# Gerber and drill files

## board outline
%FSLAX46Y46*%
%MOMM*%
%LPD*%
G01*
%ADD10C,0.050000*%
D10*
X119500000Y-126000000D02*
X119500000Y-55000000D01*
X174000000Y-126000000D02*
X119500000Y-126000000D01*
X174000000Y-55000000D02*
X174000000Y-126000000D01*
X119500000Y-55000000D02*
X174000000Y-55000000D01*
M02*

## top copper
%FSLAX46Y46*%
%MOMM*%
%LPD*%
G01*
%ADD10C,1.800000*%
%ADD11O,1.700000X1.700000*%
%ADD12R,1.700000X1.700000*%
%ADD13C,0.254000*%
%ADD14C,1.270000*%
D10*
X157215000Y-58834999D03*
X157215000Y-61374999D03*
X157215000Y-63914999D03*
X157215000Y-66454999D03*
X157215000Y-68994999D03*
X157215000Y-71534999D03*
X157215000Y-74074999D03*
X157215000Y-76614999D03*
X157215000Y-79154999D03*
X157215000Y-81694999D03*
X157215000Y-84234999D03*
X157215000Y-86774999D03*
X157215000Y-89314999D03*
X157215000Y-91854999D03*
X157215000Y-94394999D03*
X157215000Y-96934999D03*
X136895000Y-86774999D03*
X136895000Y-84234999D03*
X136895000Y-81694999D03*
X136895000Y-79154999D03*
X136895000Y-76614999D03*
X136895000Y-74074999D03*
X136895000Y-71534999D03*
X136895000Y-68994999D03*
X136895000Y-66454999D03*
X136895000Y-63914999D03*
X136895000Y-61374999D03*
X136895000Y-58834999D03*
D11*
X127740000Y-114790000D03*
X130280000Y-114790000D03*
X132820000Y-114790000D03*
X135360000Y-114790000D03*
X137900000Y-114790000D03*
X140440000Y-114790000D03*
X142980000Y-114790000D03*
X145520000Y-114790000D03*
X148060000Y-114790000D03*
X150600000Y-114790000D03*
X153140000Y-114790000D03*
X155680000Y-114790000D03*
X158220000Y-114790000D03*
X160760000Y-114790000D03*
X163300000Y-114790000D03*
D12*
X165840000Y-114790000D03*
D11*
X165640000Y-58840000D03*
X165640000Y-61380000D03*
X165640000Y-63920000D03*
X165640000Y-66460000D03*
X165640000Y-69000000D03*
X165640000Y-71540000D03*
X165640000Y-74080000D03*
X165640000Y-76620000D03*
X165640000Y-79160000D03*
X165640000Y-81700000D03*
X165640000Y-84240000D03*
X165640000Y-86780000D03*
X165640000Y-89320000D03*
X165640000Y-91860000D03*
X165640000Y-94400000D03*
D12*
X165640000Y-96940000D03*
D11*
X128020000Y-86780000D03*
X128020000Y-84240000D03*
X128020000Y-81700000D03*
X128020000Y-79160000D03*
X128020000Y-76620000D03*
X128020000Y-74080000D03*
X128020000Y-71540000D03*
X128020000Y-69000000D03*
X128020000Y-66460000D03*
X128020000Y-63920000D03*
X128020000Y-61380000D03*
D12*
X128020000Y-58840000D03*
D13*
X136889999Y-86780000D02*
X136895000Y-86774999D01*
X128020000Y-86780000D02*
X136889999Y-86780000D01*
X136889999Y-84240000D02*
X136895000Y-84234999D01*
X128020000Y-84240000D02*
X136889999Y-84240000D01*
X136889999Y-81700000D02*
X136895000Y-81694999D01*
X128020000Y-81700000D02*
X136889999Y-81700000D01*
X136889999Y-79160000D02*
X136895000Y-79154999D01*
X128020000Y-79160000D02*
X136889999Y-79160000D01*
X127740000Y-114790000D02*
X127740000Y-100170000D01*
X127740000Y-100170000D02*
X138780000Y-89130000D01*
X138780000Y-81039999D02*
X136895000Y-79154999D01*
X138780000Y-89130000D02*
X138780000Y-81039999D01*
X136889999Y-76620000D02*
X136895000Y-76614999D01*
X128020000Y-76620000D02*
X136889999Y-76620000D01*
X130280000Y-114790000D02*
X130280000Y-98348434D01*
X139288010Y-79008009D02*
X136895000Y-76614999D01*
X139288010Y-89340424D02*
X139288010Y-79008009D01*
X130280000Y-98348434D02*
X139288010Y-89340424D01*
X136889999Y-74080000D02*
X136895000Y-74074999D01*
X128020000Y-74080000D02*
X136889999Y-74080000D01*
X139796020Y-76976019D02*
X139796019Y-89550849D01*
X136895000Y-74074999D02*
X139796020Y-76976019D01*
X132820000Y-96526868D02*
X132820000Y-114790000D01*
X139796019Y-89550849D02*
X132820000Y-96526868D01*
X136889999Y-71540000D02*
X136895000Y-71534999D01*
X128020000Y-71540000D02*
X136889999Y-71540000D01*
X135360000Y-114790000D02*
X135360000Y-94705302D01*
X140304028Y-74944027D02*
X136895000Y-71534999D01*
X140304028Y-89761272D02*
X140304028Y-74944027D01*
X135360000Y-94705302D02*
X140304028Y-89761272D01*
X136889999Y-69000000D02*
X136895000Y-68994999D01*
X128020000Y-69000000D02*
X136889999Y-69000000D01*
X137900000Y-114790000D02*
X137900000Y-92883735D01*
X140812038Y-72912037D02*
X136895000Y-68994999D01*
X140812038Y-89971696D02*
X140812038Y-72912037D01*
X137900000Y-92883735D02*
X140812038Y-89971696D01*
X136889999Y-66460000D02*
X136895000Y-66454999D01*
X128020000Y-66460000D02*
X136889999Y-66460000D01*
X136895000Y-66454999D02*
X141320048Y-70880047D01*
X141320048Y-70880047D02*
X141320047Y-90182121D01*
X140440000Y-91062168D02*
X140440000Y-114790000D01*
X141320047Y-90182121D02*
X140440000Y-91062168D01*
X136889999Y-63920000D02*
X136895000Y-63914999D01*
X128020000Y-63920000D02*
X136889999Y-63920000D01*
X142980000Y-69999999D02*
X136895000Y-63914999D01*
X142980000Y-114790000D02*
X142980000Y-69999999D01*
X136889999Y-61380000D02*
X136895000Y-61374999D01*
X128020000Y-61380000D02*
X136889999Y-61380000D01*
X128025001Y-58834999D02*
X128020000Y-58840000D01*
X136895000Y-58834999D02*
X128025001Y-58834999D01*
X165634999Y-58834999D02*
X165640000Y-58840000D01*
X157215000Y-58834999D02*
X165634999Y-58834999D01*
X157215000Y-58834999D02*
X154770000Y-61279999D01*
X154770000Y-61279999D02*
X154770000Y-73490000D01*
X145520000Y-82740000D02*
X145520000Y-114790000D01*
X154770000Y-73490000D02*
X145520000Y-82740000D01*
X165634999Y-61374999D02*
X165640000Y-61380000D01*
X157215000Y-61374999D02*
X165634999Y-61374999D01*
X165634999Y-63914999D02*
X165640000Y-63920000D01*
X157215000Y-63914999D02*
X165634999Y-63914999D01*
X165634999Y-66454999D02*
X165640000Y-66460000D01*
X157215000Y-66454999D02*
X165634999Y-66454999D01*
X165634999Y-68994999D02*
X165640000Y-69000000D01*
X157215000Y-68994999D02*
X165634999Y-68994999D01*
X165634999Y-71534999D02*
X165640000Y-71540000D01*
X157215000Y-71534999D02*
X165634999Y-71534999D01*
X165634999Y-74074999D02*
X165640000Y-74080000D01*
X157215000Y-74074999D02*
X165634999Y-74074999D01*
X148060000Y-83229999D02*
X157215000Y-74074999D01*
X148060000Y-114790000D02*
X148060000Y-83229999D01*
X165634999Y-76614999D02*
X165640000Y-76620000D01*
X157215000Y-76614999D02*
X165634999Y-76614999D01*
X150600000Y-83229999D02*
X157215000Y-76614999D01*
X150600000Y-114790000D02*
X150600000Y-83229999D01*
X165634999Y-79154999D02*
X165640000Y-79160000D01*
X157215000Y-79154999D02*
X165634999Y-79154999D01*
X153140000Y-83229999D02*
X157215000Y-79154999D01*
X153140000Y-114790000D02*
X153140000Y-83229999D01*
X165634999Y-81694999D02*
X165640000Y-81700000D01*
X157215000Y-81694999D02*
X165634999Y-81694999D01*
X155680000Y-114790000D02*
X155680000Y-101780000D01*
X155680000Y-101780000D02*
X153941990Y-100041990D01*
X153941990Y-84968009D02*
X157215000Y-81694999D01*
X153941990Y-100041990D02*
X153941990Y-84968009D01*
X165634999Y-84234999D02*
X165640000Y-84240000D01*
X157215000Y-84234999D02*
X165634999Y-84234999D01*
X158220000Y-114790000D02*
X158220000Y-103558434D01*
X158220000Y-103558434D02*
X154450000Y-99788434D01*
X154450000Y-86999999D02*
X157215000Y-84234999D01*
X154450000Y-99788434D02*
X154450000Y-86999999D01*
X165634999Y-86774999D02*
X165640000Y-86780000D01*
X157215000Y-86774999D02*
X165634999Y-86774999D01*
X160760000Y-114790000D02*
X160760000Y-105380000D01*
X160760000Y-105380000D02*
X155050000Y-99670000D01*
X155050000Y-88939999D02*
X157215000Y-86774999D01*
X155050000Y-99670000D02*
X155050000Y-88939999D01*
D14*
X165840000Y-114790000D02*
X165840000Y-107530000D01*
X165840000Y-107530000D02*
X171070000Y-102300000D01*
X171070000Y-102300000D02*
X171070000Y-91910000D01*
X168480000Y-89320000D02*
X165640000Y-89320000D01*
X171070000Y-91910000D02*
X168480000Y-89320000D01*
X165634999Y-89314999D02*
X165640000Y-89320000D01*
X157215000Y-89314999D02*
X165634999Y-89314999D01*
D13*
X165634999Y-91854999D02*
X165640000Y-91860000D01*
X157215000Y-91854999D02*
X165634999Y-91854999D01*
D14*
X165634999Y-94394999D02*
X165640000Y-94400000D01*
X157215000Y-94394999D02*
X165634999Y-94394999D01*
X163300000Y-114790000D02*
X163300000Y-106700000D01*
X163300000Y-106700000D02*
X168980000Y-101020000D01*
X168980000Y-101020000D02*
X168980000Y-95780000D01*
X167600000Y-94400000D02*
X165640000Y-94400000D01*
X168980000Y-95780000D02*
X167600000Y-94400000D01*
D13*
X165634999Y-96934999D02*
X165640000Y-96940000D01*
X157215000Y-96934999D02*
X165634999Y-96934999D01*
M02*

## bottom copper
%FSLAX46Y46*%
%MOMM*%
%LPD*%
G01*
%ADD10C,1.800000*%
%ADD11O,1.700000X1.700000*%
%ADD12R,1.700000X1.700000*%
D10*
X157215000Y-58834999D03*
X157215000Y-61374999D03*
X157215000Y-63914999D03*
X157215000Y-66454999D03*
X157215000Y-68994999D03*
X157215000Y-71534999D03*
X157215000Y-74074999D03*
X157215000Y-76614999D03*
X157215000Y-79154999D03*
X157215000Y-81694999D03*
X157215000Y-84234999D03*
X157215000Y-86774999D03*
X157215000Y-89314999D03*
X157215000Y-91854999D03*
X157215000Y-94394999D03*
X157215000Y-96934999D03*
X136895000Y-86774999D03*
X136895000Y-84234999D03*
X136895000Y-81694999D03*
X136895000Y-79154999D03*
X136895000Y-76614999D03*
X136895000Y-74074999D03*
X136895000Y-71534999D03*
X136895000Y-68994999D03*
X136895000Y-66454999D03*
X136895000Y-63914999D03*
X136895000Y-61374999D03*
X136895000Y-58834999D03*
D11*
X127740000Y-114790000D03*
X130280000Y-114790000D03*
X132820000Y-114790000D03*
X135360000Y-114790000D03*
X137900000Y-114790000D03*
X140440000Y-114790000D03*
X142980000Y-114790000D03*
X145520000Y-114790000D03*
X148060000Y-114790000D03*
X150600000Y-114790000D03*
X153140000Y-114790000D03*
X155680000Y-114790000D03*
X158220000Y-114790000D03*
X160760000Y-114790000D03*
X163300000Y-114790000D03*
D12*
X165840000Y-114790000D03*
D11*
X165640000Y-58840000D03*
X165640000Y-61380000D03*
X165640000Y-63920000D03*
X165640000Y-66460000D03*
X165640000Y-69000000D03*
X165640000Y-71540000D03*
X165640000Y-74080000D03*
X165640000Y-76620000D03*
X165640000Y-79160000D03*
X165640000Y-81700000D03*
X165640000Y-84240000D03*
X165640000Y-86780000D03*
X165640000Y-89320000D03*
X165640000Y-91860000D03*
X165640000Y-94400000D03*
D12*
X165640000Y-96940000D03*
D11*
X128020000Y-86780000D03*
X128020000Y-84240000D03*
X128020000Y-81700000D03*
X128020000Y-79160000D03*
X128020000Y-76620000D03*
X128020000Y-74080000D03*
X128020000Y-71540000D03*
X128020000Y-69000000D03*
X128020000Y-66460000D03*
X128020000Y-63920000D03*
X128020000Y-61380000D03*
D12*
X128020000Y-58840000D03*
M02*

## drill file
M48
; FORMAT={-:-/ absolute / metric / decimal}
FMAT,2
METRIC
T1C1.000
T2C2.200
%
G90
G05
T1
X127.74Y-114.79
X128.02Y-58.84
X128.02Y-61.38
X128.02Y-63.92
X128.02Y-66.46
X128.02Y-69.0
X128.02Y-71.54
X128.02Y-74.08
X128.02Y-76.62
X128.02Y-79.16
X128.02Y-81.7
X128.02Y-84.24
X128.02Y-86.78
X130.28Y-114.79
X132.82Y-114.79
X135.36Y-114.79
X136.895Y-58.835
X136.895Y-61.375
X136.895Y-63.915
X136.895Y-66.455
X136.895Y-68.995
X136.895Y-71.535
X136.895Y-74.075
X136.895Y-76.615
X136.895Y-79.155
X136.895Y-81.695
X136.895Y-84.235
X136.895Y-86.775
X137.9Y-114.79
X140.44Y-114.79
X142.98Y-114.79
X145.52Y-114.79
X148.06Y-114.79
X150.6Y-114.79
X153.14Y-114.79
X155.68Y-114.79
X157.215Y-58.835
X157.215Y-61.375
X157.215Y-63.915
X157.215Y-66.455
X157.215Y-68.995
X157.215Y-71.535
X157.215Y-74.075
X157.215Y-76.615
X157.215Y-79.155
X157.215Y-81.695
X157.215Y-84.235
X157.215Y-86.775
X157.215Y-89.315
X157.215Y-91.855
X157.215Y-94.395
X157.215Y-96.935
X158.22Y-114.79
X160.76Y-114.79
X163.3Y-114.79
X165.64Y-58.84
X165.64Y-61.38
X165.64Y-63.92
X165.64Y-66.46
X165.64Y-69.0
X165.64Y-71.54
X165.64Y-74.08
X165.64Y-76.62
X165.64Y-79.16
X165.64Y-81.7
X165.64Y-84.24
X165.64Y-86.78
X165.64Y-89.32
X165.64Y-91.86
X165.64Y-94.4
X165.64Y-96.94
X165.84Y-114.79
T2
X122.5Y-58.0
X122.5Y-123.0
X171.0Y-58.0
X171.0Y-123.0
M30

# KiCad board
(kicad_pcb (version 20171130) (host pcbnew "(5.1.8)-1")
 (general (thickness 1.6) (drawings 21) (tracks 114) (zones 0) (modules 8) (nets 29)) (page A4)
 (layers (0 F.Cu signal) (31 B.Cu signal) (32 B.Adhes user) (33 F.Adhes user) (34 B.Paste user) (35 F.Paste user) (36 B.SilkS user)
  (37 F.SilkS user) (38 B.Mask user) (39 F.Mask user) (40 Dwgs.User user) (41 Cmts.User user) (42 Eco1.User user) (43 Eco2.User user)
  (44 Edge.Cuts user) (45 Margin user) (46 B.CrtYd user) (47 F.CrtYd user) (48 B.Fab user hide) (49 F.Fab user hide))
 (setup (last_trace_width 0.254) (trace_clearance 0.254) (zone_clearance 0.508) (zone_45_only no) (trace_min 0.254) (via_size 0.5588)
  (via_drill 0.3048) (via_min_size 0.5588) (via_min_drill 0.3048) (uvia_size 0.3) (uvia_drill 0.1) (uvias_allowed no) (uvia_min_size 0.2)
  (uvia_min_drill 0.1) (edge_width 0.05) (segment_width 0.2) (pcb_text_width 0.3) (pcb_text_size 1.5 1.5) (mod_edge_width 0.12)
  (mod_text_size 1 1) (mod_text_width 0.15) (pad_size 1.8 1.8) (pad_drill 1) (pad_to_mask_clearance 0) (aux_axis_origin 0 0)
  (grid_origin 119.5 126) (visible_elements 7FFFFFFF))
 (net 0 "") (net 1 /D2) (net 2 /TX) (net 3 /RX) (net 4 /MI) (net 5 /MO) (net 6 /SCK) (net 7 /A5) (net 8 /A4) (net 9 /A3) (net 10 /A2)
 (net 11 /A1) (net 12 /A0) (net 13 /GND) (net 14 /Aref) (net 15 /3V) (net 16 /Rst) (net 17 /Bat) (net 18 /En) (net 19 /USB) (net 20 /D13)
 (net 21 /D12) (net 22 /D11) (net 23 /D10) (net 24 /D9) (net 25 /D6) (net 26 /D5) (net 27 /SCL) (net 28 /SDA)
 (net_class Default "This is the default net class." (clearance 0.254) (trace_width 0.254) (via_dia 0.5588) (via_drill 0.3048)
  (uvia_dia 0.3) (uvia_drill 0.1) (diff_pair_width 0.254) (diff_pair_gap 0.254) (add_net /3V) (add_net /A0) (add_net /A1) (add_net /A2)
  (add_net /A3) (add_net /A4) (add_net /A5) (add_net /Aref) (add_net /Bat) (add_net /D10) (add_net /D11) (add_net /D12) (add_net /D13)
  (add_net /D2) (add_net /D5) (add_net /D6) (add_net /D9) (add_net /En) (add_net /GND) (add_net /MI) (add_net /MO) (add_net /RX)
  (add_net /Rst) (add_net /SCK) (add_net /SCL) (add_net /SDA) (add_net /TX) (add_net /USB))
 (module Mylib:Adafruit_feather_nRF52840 (layer F.Cu) (at 147.055 53.754999)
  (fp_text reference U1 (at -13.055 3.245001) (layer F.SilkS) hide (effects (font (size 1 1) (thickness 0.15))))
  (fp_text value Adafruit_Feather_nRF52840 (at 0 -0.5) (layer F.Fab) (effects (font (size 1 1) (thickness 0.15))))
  (pad 28 thru_hole circle (at 10.16 5.08) (size 1.8 1.8) (drill 1) (layers *.Cu *.Mask) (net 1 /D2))
  (pad 27 thru_hole circle (at 10.16 7.62) (size 1.8 1.8) (drill 1) (layers *.Cu *.Mask) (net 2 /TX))
  (pad 26 thru_hole circle (at 10.16 10.16) (size 1.8 1.8) (drill 1) (layers *.Cu *.Mask) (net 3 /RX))
  (pad 25 thru_hole circle (at 10.16 12.7) (size 1.8 1.8) (drill 1) (layers *.Cu *.Mask) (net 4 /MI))
  (pad 24 thru_hole circle (at 10.16 15.24) (size 1.8 1.8) (drill 1) (layers *.Cu *.Mask) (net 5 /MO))
  (pad 23 thru_hole circle (at 10.16 17.78) (size 1.8 1.8) (drill 1) (layers *.Cu *.Mask) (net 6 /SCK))
  (pad 22 thru_hole circle (at 10.16 20.32) (size 1.8 1.8) (drill 1) (layers *.Cu *.Mask) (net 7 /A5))
  (pad 21 thru_hole circle (at 10.16 22.86) (size 1.8 1.8) (drill 1) (layers *.Cu *.Mask) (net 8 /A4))
  (pad 20 thru_hole circle (at 10.16 25.4) (size 1.8 1.8) (drill 1) (layers *.Cu *.Mask) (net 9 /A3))
  (pad 19 thru_hole circle (at 10.16 27.94) (size 1.8 1.8) (drill 1) (layers *.Cu *.Mask) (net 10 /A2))
  (pad 18 thru_hole circle (at 10.16 30.48) (size 1.8 1.8) (drill 1) (layers *.Cu *.Mask) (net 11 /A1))
  (pad 17 thru_hole circle (at 10.16 33.02) (size 1.8 1.8) (drill 1) (layers *.Cu *.Mask) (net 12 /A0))
  (pad 16 thru_hole circle (at 10.16 35.56) (size 1.8 1.8) (drill 1) (layers *.Cu *.Mask) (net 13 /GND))
  (pad 15 thru_hole circle (at 10.16 38.1) (size 1.8 1.8) (drill 1) (layers *.Cu *.Mask) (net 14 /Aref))
  (pad 14 thru_hole circle (at 10.16 40.64) (size 1.8 1.8) (drill 1) (layers *.Cu *.Mask) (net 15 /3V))
  (pad 13 thru_hole circle (at 10.16 43.18) (size 1.8 1.8) (drill 1) (layers *.Cu *.Mask) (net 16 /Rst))
  (pad 12 thru_hole circle (at -10.16 33.02) (size 1.8 1.8) (drill 1) (layers *.Cu *.Mask) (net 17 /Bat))
  (pad 11 thru_hole circle (at -10.16 30.48) (size 1.8 1.8) (drill 1) (layers *.Cu *.Mask) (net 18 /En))
  (pad 10 thru_hole circle (at -10.16 27.94) (size 1.8 1.8) (drill 1) (layers *.Cu *.Mask) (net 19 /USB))
  (pad 9 thru_hole circle (at -10.16 25.4) (size 1.8 1.8) (drill 1) (layers *.Cu *.Mask) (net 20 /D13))
  (pad 8 thru_hole circle (at -10.16 22.86) (size 1.8 1.8) (drill 1) (layers *.Cu *.Mask) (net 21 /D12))
  (pad 7 thru_hole circle (at -10.16 20.32) (size 1.8 1.8) (drill 1) (layers *.Cu *.Mask) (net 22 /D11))
  (pad 6 thru_hole circle (at -10.16 17.78) (size 1.8 1.8) (drill 1) (layers *.Cu *.Mask) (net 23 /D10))
  (pad 5 thru_hole circle (at -10.16 15.24) (size 1.8 1.8) (drill 1) (layers *.Cu *.Mask) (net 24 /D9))
  (pad 4 thru_hole circle (at -10.16 12.7) (size 1.8 1.8) (drill 1) (layers *.Cu *.Mask) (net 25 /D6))
  (pad 3 thru_hole circle (at -10.16 10.16) (size 1.8 1.8) (drill 1) (layers *.Cu *.Mask) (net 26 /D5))
  (pad 2 thru_hole circle (at -10.16 7.62) (size 1.8 1.8) (drill 1) (layers *.Cu *.Mask) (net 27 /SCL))
  (pad 1 thru_hole circle (at -10.16 5.08) (size 1.8 1.8) (drill 1) (layers *.Cu *.Mask) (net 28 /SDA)))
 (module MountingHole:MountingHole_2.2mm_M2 (layer F.Cu) (at 171 123)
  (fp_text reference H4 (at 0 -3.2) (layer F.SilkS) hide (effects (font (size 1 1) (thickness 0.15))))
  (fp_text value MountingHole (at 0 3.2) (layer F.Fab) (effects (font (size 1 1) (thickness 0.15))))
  (pad 1 np_thru_hole circle (at 0 0) (size 2.2 2.2) (drill 2.2) (layers *.Cu *.Mask)))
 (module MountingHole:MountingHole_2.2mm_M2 (layer F.Cu) (at 171 58)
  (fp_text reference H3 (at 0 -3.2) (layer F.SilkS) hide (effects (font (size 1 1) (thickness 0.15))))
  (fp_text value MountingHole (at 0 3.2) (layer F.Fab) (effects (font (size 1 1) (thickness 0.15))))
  (pad 1 np_thru_hole circle (at 0 0) (size 2.2 2.2) (drill 2.2) (layers *.Cu *.Mask)))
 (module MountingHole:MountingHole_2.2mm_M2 (layer F.Cu) (at 122.5 123)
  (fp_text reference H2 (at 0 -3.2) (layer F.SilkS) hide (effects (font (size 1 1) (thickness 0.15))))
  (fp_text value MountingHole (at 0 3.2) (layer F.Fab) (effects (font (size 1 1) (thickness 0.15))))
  (pad 1 np_thru_hole circle (at 0 0) (size 2.2 2.2) (drill 2.2) (layers *.Cu *.Mask)))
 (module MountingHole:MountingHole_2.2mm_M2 (layer F.Cu) (at 122.5 58)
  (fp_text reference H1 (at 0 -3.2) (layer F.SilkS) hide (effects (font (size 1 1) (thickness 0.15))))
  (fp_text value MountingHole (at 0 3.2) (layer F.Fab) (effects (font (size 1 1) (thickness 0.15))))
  (pad 1 np_thru_hole circle (at 0 0) (size 2.2 2.2) (drill 2.2) (layers *.Cu *.Mask)))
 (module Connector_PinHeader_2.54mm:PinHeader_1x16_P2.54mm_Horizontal (layer F.Cu) (at 165.84 114.79 270)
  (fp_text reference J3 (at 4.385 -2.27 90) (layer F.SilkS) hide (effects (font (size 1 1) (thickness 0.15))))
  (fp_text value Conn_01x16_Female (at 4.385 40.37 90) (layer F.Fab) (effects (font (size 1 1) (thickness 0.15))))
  (pad 16 thru_hole oval (at 0 38.1 270) (size 1.7 1.7) (drill 1) (layers *.Cu *.Mask) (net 20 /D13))
  (pad 15 thru_hole oval (at 0 35.56 270) (size 1.7 1.7) (drill 1) (layers *.Cu *.Mask) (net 21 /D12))
  (pad 14 thru_hole oval (at 0 33.02 270) (size 1.7 1.7) (drill 1) (layers *.Cu *.Mask) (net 22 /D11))
  (pad 13 thru_hole oval (at 0 30.48 270) (size 1.7 1.7) (drill 1) (layers *.Cu *.Mask) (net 23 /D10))
  (pad 12 thru_hole oval (at 0 27.94 270) (size 1.7 1.7) (drill 1) (layers *.Cu *.Mask) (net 24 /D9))
  (pad 11 thru_hole oval (at 0 25.4 270) (size 1.7 1.7) (drill 1) (layers *.Cu *.Mask) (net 25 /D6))
  (pad 10 thru_hole oval (at 0 22.86 270) (size 1.7 1.7) (drill 1) (layers *.Cu *.Mask) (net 26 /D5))
  (pad 9 thru_hole oval (at 0 20.32 270) (size 1.7 1.7) (drill 1) (layers *.Cu *.Mask) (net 1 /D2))
  (pad 8 thru_hole oval (at 0 17.78 270) (size 1.7 1.7) (drill 1) (layers *.Cu *.Mask) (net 7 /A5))
  (pad 7 thru_hole oval (at 0 15.24 270) (size 1.7 1.7) (drill 1) (layers *.Cu *.Mask) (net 8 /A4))
  (pad 6 thru_hole oval (at 0 12.7 270) (size 1.7 1.7) (drill 1) (layers *.Cu *.Mask) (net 9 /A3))
  (pad 5 thru_hole oval (at 0 10.16 270) (size 1.7 1.7) (drill 1) (layers *.Cu *.Mask) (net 10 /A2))
  (pad 4 thru_hole oval (at 0 7.62 270) (size 1.7 1.7) (drill 1) (layers *.Cu *.Mask) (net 11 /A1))
  (pad 3 thru_hole oval (at 0 5.08 270) (size 1.7 1.7) (drill 1) (layers *.Cu *.Mask) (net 12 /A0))
  (pad 2 thru_hole oval (at 0 2.54 270) (size 1.7 1.7) (drill 1) (layers *.Cu *.Mask) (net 15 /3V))
  (pad 1 thru_hole rect (at 0 0 270) (size 1.7 1.7) (drill 1) (layers *.Cu *.Mask) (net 13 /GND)))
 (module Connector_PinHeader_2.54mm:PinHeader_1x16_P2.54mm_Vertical (layer F.Cu) (at 165.64 96.94 180)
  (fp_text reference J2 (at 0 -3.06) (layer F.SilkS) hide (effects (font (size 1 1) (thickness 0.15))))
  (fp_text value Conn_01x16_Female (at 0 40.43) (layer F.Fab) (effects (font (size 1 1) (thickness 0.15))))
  (pad 16 thru_hole oval (at 0 38.1 180) (size 1.7 1.7) (drill 1) (layers *.Cu *.Mask) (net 1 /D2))
  (pad 15 thru_hole oval (at 0 35.56 180) (size 1.7 1.7) (drill 1) (layers *.Cu *.Mask) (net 2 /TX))
  (pad 14 thru_hole oval (at 0 33.02 180) (size 1.7 1.7) (drill 1) (layers *.Cu *.Mask) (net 3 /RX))
  (pad 13 thru_hole oval (at 0 30.48 180) (size 1.7 1.7) (drill 1) (layers *.Cu *.Mask) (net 4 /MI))
  (pad 12 thru_hole oval (at 0 27.94 180) (size 1.7 1.7) (drill 1) (layers *.Cu *.Mask) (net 5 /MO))
  (pad 11 thru_hole oval (at 0 25.4 180) (size 1.7 1.7) (drill 1) (layers *.Cu *.Mask) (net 6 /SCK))
  (pad 10 thru_hole oval (at 0 22.86 180) (size 1.7 1.7) (drill 1) (layers *.Cu *.Mask) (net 7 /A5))
  (pad 9 thru_hole oval (at 0 20.32 180) (size 1.7 1.7) (drill 1) (layers *.Cu *.Mask) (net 8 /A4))
  (pad 8 thru_hole oval (at 0 17.78 180) (size 1.7 1.7) (drill 1) (layers *.Cu *.Mask) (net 9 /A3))
  (pad 7 thru_hole oval (at 0 15.24 180) (size 1.7 1.7) (drill 1) (layers *.Cu *.Mask) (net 10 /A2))
  (pad 6 thru_hole oval (at 0 12.7 180) (size 1.7 1.7) (drill 1) (layers *.Cu *.Mask) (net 11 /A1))
  (pad 5 thru_hole oval (at 0 10.16 180) (size 1.7 1.7) (drill 1) (layers *.Cu *.Mask) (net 12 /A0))
  (pad 4 thru_hole oval (at 0 7.62 180) (size 1.7 1.7) (drill 1) (layers *.Cu *.Mask) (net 13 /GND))
  (pad 3 thru_hole oval (at 0 5.08 180) (size 1.7 1.7) (drill 1) (layers *.Cu *.Mask) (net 14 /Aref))
  (pad 2 thru_hole oval (at 0 2.54 180) (size 1.7 1.7) (drill 1) (layers *.Cu *.Mask) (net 15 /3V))
  (pad 1 thru_hole rect (at 0 0 180) (size 1.7 1.7) (drill 1) (layers *.Cu *.Mask) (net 16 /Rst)))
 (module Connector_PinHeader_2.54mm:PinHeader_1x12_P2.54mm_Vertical (layer F.Cu) (at 128.02 58.84)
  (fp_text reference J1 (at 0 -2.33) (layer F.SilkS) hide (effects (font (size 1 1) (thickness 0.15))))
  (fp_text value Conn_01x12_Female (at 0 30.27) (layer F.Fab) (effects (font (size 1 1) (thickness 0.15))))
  (pad 12 thru_hole oval (at 0 27.94) (size 1.7 1.7) (drill 1) (layers *.Cu *.Mask) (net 17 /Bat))
  (pad 11 thru_hole oval (at 0 25.4) (size 1.7 1.7) (drill 1) (layers *.Cu *.Mask) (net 18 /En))
  (pad 10 thru_hole oval (at 0 22.86) (size 1.7 1.7) (drill 1) (layers *.Cu *.Mask) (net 19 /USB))
  (pad 9 thru_hole oval (at 0 20.32) (size 1.7 1.7) (drill 1) (layers *.Cu *.Mask) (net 20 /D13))
  (pad 8 thru_hole oval (at 0 17.78) (size 1.7 1.7) (drill 1) (layers *.Cu *.Mask) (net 21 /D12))
  (pad 7 thru_hole oval (at 0 15.24) (size 1.7 1.7) (drill 1) (layers *.Cu *.Mask) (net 22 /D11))
  (pad 6 thru_hole oval (at 0 12.7) (size 1.7 1.7) (drill 1) (layers *.Cu *.Mask) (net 23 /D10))
  (pad 5 thru_hole oval (at 0 10.16) (size 1.7 1.7) (drill 1) (layers *.Cu *.Mask) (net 24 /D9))
  (pad 4 thru_hole oval (at 0 7.62) (size 1.7 1.7) (drill 1) (layers *.Cu *.Mask) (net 25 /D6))
  (pad 3 thru_hole oval (at 0 5.08) (size 1.7 1.7) (drill 1) (layers *.Cu *.Mask) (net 26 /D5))
  (pad 2 thru_hole oval (at 0 2.54) (size 1.7 1.7) (drill 1) (layers *.Cu *.Mask) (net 27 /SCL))
  (pad 1 thru_hole rect (at 0 0) (size 1.7 1.7) (drill 1) (layers *.Cu *.Mask) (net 28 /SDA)))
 (gr_line (start 119.5 126) (end 119.5 55) (layer Edge.Cuts) (width 0.05))
 (gr_line (start 174 126) (end 119.5 126) (layer Edge.Cuts) (width 0.05))
 (gr_line (start 174 55) (end 174 126) (layer Edge.Cuts) (width 0.05))
 (gr_line (start 119.5 55) (end 174 55) (layer Edge.Cuts) (width 0.05))
 (segment (start 136.889999 86.78) (end 136.895 86.774999) (width 0.254) (layer F.Cu) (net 17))
 (segment (start 128.02 86.78) (end 136.889999 86.78) (width 0.254) (layer F.Cu) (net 17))
 (segment (start 136.889999 84.24) (end 136.895 84.234999) (width 0.254) (layer F.Cu) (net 18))
 (segment (start 128.02 84.24) (end 136.889999 84.24) (width 0.254) (layer F.Cu) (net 18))
 (segment (start 136.889999 81.7) (end 136.895 81.694999) (width 0.254) (layer F.Cu) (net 19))
 (segment (start 128.02 81.7) (end 136.889999 81.7) (width 0.254) (layer F.Cu) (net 19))
 (segment (start 136.889999 79.16) (end 136.895 79.154999) (width 0.254) (layer F.Cu) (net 20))
 (segment (start 128.02 79.16) (end 136.889999 79.16) (width 0.254) (layer F.Cu) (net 20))
 (segment (start 127.74 114.79) (end 127.74 100.17) (width 0.254) (layer F.Cu) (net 20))
 (segment (start 127.74 100.17) (end 138.78 89.13) (width 0.254) (layer F.Cu) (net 20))
 (segment (start 138.78 81.039999) (end 136.895 79.154999) (width 0.254) (layer F.Cu) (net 20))
 (segment (start 138.78 89.13) (end 138.78 81.039999) (width 0.254) (layer F.Cu) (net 20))
 (segment (start 136.889999 76.62) (end 136.895 76.614999) (width 0.254) (layer F.Cu) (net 21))
 (segment (start 128.02 76.62) (end 136.889999 76.62) (width 0.254) (layer F.Cu) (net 21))
 (segment (start 130.28 114.79) (end 130.28 98.348434) (width 0.254) (layer F.Cu) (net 21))
 (segment (start 139.28801 79.008009) (end 136.895 76.614999) (width 0.254) (layer F.Cu) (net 21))
 (segment (start 139.28801 89.340424) (end 139.28801 79.008009) (width 0.254) (layer F.Cu) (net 21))
 (segment (start 130.28 98.348434) (end 139.28801 89.340424) (width 0.254) (layer F.Cu) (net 21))
 (segment (start 136.889999 74.08) (end 136.895 74.074999) (width 0.254) (layer F.Cu) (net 22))
 (segment (start 128.02 74.08) (end 136.889999 74.08) (width 0.254) (layer F.Cu) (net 22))
 (segment (start 139.79602 76.976019) (end 139.796019 89.550849) (width 0.254) (layer F.Cu) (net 22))
 (segment (start 136.895 74.074999) (end 139.79602 76.976019) (width 0.254) (layer F.Cu) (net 22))
 (segment (start 132.82 96.526868) (end 132.82 114.79) (width 0.254) (layer F.Cu) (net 22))
 (segment (start 139.796019 89.550849) (end 132.82 96.526868) (width 0.254) (layer F.Cu) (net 22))
 (segment (start 136.889999 71.54) (end 136.895 71.534999) (width 0.254) (layer F.Cu) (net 23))
 (segment (start 128.02 71.54) (end 136.889999 71.54) (width 0.254) (layer F.Cu) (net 23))
 (segment (start 135.36 114.79) (end 135.36 94.705302) (width 0.254) (layer F.Cu) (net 23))
 (segment (start 140.304028 74.944027) (end 136.895 71.534999) (width 0.254) (layer F.Cu) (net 23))
 (segment (start 140.304028 89.761272) (end 140.304028 74.944027) (width 0.254) (layer F.Cu) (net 23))
 (segment (start 135.36 94.705302) (end 140.304028 89.761272) (width 0.254) (layer F.Cu) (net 23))
 (segment (start 136.889999 69) (end 136.895 68.994999) (width 0.254) (layer F.Cu) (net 24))
 (segment (start 128.02 69) (end 136.889999 69) (width 0.254) (layer F.Cu) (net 24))
 (segment (start 137.9 114.79) (end 137.9 92.883735) (width 0.254) (layer F.Cu) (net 24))
 (segment (start 140.812038 72.912037) (end 136.895 68.994999) (width 0.254) (layer F.Cu) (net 24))
 (segment (start 140.812038 89.971696) (end 140.812038 72.912037) (width 0.254) (layer F.Cu) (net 24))
 (segment (start 137.9 92.883735) (end 140.812038 89.971696) (width 0.254) (layer F.Cu) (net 24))
 (segment (start 136.889999 66.46) (end 136.895 66.454999) (width 0.254) (layer F.Cu) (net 25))
 (segment (start 128.02 66.46) (end 136.889999 66.46) (width 0.254) (layer F.Cu) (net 25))
 (segment (start 136.895 66.454999) (end 141.320048 70.880047) (width 0.254) (layer F.Cu) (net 25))
 (segment (start 141.320048 70.880047) (end 141.320047 90.182121) (width 0.254) (layer F.Cu) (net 25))
 (segment (start 140.44 91.062168) (end 140.44 114.79) (width 0.254) (layer F.Cu) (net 25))
 (segment (start 141.320047 90.182121) (end 140.44 91.062168) (width 0.254) (layer F.Cu) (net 25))
 (segment (start 136.889999 63.92) (end 136.895 63.914999) (width 0.254) (layer F.Cu) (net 26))
 (segment (start 128.02 63.92) (end 136.889999 63.92) (width 0.254) (layer F.Cu) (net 26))
 (segment (start 142.98 69.999999) (end 136.895 63.914999) (width 0.254) (layer F.Cu) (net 26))
 (segment (start 142.98 114.79) (end 142.98 69.999999) (width 0.254) (layer F.Cu) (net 26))
 (segment (start 136.889999 61.38) (end 136.895 61.374999) (width 0.254) (layer F.Cu) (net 27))
 (segment (start 128.02 61.38) (end 136.889999 61.38) (width 0.254) (layer F.Cu) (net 27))
 (segment (start 128.025001 58.834999) (end 128.02 58.84) (width 0.254) (layer F.Cu) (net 28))
 (segment (start 136.895 58.834999) (end 128.025001 58.834999) (width 0.254) (layer F.Cu) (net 28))
 (segment (start 165.634999 58.834999) (end 165.64 58.84) (width 0.254) (layer F.Cu) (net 1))
 (segment (start 157.215 58.834999) (end 165.634999 58.834999) (width 0.254) (layer F.Cu) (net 1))
 (segment (start 157.215 58.834999) (end 154.77 61.279999) (width 0.254) (layer F.Cu) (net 1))
 (segment (start 154.77 61.279999) (end 154.77 73.49) (width 0.254) (layer F.Cu) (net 1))
 (segment (start 145.52 82.74) (end 145.52 114.79) (width 0.254) (layer F.Cu) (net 1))
 (segment (start 154.77 73.49) (end 145.52 82.74) (width 0.254) (layer F.Cu) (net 1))
 (segment (start 165.634999 61.374999) (end 165.64 61.38) (width 0.254) (layer F.Cu) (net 2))
 (segment (start 157.215 61.374999) (end 165.634999 61.374999) (width 0.254) (layer F.Cu) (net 2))
 (segment (start 165.634999 63.914999) (end 165.64 63.92) (width 0.254) (layer F.Cu) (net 3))
 (segment (start 157.215 63.914999) (end 165.634999 63.914999) (width 0.254) (layer F.Cu) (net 3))
 (segment (start 165.634999 66.454999) (end 165.64 66.46) (width 0.254) (layer F.Cu) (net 4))
 (segment (start 157.215 66.454999) (end 165.634999 66.454999) (width 0.254) (layer F.Cu) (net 4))
 (segment (start 165.634999 68.994999) (end 165.64 69) (width 0.254) (layer F.Cu) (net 5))
 (segment (start 157.215 68.994999) (end 165.634999 68.994999) (width 0.254) (layer F.Cu) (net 5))
 (segment (start 165.634999 71.534999) (end 165.64 71.54) (width 0.254) (layer F.Cu) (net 6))
 (segment (start 157.215 71.534999) (end 165.634999 71.534999) (width 0.254) (layer F.Cu) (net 6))
 (segment (start 165.634999 74.074999) (end 165.64 74.08) (width 0.254) (layer F.Cu) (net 7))
 (segment (start 157.215 74.074999) (end 165.634999 74.074999) (width 0.254) (layer F.Cu) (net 7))
 (segment (start 148.06 83.229999) (end 157.215 74.074999) (width 0.254) (layer F.Cu) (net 7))
 (segment (start 148.06 114.79) (end 148.06 83.229999) (width 0.254) (layer F.Cu) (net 7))
 (segment (start 165.634999 76.614999) (end 165.64 76.62) (width 0.254) (layer F.Cu) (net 8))
 (segment (start 157.215 76.614999) (end 165.634999 76.614999) (width 0.254) (layer F.Cu) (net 8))
 (segment (start 150.6 83.229999) (end 157.215 76.614999) (width 0.254) (layer F.Cu) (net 8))
 (segment (start 150.6 114.79) (end 150.6 83.229999) (width 0.254) (layer F.Cu) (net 8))
 (segment (start 165.634999 79.154999) (end 165.64 79.16) (width 0.254) (layer F.Cu) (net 9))
 (segment (start 157.215 79.154999) (end 165.634999 79.154999) (width 0.254) (layer F.Cu) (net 9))
 (segment (start 153.14 83.229999) (end 157.215 79.154999) (width 0.254) (layer F.Cu) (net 9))
 (segment (start 153.14 114.79) (end 153.14 83.229999) (width 0.254) (layer F.Cu) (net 9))
 (segment (start 165.634999 81.694999) (end 165.64 81.7) (width 0.254) (layer F.Cu) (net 10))
 (segment (start 157.215 81.694999) (end 165.634999 81.694999) (width 0.254) (layer F.Cu) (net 10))
 (segment (start 155.68 114.79) (end 155.68 101.78) (width 0.254) (layer F.Cu) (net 10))
 (segment (start 155.68 101.78) (end 153.94199 100.04199) (width 0.254) (layer F.Cu) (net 10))
 (segment (start 153.94199 84.968009) (end 157.215 81.694999) (width 0.254) (layer F.Cu) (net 10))
 (segment (start 153.94199 100.04199) (end 153.94199 84.968009) (width 0.254) (layer F.Cu) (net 10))
 (segment (start 165.634999 84.234999) (end 165.64 84.24) (width 0.254) (layer F.Cu) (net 11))
 (segment (start 157.215 84.234999) (end 165.634999 84.234999) (width 0.254) (layer F.Cu) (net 11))
 (segment (start 158.22 114.79) (end 158.22 103.558434) (width 0.254) (layer F.Cu) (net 11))
 (segment (start 158.22 103.558434) (end 154.45 99.788434) (width 0.254) (layer F.Cu) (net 11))
 (segment (start 154.45 86.999999) (end 157.215 84.234999) (width 0.254) (layer F.Cu) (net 11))
 (segment (start 154.45 99.788434) (end 154.45 86.999999) (width 0.254) (layer F.Cu) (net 11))
 (segment (start 165.634999 86.774999) (end 165.64 86.78) (width 0.254) (layer F.Cu) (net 12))
 (segment (start 157.215 86.774999) (end 165.634999 86.774999) (width 0.254) (layer F.Cu) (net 12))
 (segment (start 160.76 114.79) (end 160.76 105.38) (width 0.254) (layer F.Cu) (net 12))
 (segment (start 160.76 105.38) (end 155.05 99.67) (width 0.254) (layer F.Cu) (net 12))
 (segment (start 155.05 88.939999) (end 157.215 86.774999) (width 0.254) (layer F.Cu) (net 12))
 (segment (start 155.05 99.67) (end 155.05 88.939999) (width 0.254) (layer F.Cu) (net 12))
 (segment (start 165.84 114.79) (end 165.84 107.53) (width 1.27) (layer F.Cu) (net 13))
 (segment (start 165.84 107.53) (end 171.07 102.3) (width 1.27) (layer F.Cu) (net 13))
 (segment (start 171.07 102.3) (end 171.07 91.91) (width 1.27) (layer F.Cu) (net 13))
 (segment (start 168.48 89.32) (end 165.64 89.32) (width 1.27) (layer F.Cu) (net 13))
 (segment (start 171.07 91.91) (end 168.48 89.32) (width 1.27) (layer F.Cu) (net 13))
 (segment (start 165.634999 89.314999) (end 165.64 89.32) (width 1.27) (layer F.Cu) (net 13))
 (segment (start 157.215 89.314999) (end 165.634999 89.314999) (width 1.27) (layer F.Cu) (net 13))
 (segment (start 165.634999 91.854999) (end 165.64 91.86) (width 0.254) (layer F.Cu) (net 14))
 (segment (start 157.215 91.854999) (end 165.634999 91.854999) (width 0.254) (layer F.Cu) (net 14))
 (segment (start 165.634999 94.394999) (end 165.64 94.4) (width 1.27) (layer F.Cu) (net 15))
 (segment (start 157.215 94.394999) (end 165.634999 94.394999) (width 1.27) (layer F.Cu) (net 15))
 (segment (start 163.3 114.79) (end 163.3 106.7) (width 1.27) (layer F.Cu) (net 15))
 (segment (start 163.3 106.7) (end 168.98 101.02) (width 1.27) (layer F.Cu) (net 15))
 (segment (start 168.98 101.02) (end 168.98 95.78) (width 1.27) (layer F.Cu) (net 15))
 (segment (start 167.6 94.4) (end 165.64 94.4) (width 1.27) (layer F.Cu) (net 15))
 (segment (start 168.98 95.78) (end 167.6 94.4) (width 1.27) (layer F.Cu) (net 15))
 (segment (start 165.634999 96.934999) (end 165.64 96.94) (width 0.254) (layer F.Cu) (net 16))
 (segment (start 157.215 96.934999) (end 165.634999 96.934999) (width 0.254) (layer F.Cu) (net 16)))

